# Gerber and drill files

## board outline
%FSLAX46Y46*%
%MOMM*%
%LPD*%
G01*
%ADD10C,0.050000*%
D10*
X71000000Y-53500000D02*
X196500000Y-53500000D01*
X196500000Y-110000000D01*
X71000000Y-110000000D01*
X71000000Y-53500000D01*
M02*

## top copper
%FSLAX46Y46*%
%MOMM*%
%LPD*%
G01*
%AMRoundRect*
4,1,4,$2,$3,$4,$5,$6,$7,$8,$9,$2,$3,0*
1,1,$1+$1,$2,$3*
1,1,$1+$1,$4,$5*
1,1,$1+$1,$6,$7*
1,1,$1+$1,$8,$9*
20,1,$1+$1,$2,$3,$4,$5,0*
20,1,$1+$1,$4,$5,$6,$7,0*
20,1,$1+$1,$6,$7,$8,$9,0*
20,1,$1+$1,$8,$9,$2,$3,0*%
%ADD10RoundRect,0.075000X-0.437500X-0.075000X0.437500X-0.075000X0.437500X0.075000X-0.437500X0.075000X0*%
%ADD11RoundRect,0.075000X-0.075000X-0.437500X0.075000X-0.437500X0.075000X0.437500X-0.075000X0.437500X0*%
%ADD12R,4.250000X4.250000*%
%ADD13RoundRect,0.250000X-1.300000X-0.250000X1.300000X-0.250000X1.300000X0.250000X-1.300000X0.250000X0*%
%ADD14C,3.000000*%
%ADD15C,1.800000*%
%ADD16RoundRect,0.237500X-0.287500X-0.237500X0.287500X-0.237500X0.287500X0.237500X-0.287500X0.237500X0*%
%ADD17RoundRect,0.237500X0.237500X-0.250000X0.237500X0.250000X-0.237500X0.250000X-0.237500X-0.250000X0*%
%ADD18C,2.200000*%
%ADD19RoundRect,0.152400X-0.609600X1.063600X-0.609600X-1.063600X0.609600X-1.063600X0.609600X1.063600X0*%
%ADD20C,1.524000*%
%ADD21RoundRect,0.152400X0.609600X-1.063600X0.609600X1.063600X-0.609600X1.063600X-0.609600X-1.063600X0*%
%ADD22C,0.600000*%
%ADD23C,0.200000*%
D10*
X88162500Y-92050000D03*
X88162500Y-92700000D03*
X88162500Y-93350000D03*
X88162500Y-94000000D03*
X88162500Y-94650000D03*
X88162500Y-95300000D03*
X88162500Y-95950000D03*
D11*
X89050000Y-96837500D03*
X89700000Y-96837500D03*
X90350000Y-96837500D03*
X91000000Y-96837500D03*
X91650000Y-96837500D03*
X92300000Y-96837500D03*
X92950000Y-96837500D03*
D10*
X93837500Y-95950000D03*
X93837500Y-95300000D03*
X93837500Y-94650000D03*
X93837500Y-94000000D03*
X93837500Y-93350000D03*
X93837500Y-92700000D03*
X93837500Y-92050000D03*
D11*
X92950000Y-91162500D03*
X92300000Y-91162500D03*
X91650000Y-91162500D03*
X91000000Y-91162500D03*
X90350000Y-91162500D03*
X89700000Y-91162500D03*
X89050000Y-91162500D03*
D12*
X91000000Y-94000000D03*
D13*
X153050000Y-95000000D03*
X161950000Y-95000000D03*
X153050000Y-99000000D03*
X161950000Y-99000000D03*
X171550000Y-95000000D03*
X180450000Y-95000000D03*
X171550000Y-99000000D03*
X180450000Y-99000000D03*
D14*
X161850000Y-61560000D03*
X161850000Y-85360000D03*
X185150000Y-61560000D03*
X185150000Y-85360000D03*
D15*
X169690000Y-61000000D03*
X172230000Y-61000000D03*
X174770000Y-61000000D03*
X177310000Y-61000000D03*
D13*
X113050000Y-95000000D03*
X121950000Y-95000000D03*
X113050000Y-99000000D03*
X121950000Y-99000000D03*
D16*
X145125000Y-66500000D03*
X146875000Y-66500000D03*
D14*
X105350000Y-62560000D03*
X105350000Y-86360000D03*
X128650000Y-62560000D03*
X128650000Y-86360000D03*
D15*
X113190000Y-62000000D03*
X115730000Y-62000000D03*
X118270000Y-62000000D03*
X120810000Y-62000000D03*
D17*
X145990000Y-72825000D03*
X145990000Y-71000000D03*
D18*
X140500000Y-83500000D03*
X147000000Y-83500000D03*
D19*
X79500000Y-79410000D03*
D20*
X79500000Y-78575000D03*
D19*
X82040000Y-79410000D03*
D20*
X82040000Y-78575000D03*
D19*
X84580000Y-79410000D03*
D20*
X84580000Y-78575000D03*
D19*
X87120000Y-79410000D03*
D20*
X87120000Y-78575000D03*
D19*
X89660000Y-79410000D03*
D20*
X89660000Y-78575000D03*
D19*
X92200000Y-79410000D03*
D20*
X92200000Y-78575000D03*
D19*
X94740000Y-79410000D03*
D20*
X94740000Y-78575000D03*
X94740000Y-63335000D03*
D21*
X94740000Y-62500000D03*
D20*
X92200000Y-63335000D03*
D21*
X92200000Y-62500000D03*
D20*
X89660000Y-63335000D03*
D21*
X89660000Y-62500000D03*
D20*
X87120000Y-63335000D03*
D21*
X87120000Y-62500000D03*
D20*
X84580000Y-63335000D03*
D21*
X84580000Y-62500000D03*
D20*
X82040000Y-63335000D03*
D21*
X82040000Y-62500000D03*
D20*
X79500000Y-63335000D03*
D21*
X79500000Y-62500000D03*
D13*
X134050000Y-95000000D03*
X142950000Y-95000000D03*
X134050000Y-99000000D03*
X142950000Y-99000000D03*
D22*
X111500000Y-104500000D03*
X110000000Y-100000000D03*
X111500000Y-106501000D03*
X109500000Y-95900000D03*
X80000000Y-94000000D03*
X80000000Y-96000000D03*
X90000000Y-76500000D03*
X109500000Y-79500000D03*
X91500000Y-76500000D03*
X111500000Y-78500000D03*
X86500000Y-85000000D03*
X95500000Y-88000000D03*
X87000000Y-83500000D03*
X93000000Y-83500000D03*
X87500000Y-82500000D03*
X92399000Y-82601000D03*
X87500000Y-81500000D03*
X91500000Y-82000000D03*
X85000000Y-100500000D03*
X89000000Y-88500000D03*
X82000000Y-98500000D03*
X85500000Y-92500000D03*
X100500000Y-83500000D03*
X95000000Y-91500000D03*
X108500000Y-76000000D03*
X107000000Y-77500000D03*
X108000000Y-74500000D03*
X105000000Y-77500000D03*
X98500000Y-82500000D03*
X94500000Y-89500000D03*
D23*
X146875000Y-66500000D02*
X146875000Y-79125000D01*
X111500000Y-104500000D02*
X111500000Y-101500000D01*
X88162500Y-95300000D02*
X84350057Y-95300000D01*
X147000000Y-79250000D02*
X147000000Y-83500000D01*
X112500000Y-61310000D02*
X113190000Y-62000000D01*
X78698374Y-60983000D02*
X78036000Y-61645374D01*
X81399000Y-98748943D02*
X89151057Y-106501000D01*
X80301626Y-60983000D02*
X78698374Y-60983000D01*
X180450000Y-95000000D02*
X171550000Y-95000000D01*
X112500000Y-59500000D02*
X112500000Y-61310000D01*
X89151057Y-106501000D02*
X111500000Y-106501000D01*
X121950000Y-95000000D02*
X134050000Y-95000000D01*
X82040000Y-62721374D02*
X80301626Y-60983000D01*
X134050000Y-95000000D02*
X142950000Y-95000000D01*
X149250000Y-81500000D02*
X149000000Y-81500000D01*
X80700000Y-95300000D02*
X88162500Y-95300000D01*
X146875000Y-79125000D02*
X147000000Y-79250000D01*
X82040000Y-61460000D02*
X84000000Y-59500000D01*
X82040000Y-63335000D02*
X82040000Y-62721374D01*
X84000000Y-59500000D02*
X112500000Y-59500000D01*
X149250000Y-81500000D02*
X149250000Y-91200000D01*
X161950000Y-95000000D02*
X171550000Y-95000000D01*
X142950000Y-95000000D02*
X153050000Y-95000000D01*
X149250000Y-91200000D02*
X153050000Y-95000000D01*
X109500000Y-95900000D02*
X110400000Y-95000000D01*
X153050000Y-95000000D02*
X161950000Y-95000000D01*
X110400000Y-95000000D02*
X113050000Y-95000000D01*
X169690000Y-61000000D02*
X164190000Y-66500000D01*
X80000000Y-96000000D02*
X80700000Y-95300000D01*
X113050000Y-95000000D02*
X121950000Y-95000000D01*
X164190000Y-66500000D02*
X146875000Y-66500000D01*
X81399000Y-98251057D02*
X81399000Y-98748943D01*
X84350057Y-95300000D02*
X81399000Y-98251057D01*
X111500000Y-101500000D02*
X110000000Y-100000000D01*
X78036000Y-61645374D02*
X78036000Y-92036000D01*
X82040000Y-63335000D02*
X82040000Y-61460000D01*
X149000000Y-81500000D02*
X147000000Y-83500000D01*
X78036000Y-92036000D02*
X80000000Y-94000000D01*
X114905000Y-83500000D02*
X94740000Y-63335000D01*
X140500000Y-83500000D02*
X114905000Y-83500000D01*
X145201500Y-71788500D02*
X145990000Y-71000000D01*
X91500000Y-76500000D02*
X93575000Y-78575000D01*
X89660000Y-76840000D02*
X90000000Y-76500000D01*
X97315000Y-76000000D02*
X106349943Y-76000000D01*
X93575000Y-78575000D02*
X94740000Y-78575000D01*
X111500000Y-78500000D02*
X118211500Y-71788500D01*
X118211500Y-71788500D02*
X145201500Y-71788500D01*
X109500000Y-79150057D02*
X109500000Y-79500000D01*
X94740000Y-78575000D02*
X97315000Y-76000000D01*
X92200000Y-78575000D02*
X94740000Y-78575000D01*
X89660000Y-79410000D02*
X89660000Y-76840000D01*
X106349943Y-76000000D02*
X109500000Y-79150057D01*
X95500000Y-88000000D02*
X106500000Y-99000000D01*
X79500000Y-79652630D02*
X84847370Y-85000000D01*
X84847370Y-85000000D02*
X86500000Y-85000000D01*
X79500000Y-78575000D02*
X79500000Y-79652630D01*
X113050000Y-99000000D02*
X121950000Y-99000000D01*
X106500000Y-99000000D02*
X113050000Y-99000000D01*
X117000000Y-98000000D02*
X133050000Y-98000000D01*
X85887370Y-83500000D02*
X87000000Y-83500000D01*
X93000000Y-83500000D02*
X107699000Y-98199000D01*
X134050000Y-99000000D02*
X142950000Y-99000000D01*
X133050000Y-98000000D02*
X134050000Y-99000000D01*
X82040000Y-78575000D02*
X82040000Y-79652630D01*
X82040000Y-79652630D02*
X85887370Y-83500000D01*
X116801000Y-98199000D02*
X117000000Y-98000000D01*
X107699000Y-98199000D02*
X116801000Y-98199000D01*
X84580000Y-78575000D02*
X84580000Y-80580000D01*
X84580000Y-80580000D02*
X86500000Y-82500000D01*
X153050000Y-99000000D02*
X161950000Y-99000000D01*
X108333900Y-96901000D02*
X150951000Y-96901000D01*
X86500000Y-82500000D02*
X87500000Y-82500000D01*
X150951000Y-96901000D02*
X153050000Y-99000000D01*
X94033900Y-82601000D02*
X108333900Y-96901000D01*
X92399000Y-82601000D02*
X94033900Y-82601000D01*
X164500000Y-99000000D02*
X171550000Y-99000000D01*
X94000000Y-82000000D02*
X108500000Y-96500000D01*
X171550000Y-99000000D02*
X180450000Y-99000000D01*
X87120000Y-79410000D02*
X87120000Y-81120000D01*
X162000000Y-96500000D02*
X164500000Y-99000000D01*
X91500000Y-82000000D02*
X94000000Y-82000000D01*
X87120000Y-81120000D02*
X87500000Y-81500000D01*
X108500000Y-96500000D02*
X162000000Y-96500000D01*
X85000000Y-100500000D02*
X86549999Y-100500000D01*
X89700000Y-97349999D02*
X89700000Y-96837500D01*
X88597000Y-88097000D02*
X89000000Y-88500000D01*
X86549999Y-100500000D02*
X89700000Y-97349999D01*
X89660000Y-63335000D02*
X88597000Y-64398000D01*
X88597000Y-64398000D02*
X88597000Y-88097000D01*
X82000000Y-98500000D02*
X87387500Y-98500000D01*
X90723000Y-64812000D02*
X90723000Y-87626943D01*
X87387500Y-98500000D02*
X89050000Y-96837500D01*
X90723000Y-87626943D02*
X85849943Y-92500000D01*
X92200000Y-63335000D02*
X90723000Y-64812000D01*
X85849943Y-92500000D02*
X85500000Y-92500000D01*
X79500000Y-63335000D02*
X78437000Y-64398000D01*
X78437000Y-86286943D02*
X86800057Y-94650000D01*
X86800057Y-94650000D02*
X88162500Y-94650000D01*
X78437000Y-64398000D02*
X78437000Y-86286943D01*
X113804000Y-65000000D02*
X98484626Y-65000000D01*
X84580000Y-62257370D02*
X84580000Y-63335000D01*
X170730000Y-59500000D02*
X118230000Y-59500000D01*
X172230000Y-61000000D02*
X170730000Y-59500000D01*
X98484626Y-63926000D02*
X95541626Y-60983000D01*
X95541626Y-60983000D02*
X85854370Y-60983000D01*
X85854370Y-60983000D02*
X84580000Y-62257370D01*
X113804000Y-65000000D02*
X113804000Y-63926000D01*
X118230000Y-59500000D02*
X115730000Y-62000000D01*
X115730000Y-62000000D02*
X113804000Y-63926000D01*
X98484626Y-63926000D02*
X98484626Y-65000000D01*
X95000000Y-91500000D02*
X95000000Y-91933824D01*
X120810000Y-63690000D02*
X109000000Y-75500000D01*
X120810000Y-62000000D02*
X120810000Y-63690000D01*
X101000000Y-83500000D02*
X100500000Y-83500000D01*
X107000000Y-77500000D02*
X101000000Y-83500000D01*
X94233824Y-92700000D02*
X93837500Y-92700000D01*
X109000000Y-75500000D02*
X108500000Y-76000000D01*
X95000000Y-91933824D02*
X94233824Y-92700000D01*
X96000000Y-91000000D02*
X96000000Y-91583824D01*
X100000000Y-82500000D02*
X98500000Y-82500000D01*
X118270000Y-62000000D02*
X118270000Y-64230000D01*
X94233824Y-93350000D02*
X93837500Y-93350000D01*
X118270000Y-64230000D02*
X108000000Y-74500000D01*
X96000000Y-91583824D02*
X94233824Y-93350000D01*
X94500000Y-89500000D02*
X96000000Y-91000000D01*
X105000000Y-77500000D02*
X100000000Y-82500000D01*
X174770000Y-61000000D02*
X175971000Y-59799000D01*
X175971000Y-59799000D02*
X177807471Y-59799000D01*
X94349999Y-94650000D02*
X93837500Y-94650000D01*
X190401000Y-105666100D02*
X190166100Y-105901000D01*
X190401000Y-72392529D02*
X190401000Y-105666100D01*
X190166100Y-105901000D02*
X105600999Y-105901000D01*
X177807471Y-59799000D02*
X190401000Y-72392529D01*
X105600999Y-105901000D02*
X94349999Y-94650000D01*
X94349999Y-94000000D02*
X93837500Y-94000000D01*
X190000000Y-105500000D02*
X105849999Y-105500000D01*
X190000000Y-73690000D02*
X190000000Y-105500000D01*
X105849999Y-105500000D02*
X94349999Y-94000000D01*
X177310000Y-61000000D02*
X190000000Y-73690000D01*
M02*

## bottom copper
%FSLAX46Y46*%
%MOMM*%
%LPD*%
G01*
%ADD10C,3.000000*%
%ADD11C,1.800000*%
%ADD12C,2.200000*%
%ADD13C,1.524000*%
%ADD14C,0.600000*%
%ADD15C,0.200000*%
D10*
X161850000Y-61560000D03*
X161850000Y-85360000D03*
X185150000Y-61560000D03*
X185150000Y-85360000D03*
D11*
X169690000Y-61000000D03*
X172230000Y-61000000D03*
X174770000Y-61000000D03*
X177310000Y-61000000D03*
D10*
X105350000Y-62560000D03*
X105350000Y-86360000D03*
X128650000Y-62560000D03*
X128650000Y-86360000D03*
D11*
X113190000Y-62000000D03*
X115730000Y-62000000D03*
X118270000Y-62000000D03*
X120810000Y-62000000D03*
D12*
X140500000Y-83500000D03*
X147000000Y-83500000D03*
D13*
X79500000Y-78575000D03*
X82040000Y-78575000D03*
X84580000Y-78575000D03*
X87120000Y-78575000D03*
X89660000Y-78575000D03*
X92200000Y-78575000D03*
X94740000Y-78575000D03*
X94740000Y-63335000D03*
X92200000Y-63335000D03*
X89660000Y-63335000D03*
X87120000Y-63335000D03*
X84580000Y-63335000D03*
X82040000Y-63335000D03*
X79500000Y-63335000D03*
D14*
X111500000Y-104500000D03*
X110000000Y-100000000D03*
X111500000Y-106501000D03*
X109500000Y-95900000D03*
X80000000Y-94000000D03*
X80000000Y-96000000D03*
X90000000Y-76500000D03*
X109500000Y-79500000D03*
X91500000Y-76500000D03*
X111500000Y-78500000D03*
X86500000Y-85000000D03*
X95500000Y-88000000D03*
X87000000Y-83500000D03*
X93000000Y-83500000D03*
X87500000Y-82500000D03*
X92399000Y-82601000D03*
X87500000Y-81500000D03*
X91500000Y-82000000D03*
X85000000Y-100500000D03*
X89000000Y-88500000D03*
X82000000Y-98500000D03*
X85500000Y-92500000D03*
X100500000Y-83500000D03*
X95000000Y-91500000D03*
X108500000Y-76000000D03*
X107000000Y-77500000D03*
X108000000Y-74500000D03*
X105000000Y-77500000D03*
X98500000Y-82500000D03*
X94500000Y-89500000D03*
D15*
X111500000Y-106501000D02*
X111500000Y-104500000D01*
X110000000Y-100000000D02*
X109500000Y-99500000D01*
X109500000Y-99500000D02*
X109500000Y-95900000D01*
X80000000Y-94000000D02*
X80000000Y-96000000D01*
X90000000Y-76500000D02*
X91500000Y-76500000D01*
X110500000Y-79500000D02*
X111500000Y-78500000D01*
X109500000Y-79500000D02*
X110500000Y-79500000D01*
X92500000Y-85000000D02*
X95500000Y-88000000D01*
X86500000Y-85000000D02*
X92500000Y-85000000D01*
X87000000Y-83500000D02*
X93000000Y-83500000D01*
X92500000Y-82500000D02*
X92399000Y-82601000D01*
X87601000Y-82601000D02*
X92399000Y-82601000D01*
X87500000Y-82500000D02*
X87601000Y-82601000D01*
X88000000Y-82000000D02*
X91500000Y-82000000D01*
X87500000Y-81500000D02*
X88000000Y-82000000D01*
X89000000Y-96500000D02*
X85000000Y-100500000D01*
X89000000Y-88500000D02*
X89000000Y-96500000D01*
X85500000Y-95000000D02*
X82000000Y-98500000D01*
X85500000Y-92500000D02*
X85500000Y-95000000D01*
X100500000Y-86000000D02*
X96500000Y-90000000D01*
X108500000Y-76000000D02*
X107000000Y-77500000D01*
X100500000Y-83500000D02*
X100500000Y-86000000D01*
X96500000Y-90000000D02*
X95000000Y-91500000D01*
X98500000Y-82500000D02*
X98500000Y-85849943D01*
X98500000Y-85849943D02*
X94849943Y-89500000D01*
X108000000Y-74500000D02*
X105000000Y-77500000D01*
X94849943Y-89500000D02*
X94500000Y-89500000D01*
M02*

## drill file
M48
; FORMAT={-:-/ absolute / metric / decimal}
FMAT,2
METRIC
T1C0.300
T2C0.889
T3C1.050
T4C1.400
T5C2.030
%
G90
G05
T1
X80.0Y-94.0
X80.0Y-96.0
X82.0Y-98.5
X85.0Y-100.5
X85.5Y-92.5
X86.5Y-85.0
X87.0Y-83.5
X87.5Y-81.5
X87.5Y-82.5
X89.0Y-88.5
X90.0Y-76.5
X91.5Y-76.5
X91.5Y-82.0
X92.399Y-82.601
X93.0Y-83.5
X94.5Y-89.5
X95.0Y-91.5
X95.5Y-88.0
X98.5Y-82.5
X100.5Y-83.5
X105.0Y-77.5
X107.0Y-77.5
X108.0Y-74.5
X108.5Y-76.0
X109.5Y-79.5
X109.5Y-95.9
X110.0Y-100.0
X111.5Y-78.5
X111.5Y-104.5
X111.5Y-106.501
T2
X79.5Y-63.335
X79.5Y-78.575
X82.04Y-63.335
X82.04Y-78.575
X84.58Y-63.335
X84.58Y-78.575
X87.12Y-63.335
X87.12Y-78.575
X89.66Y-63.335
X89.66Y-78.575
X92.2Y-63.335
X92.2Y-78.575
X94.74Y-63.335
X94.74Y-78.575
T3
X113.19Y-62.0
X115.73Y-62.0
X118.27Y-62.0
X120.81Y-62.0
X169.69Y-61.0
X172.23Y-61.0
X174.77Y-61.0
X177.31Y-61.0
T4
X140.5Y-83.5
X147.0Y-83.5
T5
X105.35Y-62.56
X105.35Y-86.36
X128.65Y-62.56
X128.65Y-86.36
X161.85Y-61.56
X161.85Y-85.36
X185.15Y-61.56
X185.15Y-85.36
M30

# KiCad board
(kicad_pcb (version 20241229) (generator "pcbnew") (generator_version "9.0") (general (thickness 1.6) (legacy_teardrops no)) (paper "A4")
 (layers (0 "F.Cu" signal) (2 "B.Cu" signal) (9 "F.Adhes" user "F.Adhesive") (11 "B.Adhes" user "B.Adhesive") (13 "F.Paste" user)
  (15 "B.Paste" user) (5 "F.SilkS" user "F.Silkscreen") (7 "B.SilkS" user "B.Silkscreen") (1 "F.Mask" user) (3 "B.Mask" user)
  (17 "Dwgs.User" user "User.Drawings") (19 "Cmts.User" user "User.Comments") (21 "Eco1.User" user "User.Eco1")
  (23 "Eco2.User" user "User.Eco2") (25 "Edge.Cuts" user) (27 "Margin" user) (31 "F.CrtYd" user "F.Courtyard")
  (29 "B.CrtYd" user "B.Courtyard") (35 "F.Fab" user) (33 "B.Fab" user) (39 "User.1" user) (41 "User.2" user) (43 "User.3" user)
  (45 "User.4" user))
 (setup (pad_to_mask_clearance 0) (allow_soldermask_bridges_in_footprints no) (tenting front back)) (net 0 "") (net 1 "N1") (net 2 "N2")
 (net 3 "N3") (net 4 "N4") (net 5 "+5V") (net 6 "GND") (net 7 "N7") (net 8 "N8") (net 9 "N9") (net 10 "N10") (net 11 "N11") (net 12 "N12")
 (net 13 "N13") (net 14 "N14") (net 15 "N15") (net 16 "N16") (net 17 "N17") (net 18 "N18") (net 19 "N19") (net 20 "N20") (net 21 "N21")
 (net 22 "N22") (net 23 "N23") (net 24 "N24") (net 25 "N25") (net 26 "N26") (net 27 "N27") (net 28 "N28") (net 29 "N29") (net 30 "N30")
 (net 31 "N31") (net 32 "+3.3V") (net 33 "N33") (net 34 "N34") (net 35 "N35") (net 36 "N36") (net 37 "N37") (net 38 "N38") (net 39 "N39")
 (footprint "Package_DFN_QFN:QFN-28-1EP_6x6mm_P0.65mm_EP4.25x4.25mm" (layer "F.Cu") (at 91 94)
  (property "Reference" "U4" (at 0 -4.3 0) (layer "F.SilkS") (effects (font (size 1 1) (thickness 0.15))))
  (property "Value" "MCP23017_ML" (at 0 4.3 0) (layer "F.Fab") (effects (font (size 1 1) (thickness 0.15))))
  (pad "" smd roundrect (at -1.42 -1.42) (size 1.14 1.14) (layers "F.Paste") (roundrect_rratio 0.219298))
  (pad "" smd roundrect (at -1.42 0) (size 1.14 1.14) (layers "F.Paste") (roundrect_rratio 0.219298))
  (pad "" smd roundrect (at -1.42 1.42) (size 1.14 1.14) (layers "F.Paste") (roundrect_rratio 0.219298))
  (pad "" smd roundrect (at 0 -1.42) (size 1.14 1.14) (layers "F.Paste") (roundrect_rratio 0.219298))
  (pad "" smd roundrect (at 0 0) (size 1.14 1.14) (layers "F.Paste") (roundrect_rratio 0.219298))
  (pad "" smd roundrect (at 0 1.42) (size 1.14 1.14) (layers "F.Paste") (roundrect_rratio 0.219298))
  (pad "" smd roundrect (at 1.42 -1.42) (size 1.14 1.14) (layers "F.Paste") (roundrect_rratio 0.219298))
  (pad "" smd roundrect (at 1.42 0) (size 1.14 1.14) (layers "F.Paste") (roundrect_rratio 0.219298))
  (pad "" smd roundrect (at 1.42 1.42) (size 1.14 1.14) (layers "F.Paste") (roundrect_rratio 0.219298))
  (pad "1" smd roundrect (at -2.8375 -1.95) (size 1.025 0.3) (layers "F.Cu" "F.Mask" "F.Paste") (roundrect_rratio 0.25) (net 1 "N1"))
  (pad "2" smd roundrect (at -2.8375 -1.3) (size 1.025 0.3) (layers "F.Cu" "F.Mask" "F.Paste") (roundrect_rratio 0.25) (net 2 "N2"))
  (pad "3" smd roundrect (at -2.8375 -0.65) (size 1.025 0.3) (layers "F.Cu" "F.Mask" "F.Paste") (roundrect_rratio 0.25) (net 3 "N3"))
  (pad "4" smd roundrect (at -2.8375 0) (size 1.025 0.3) (layers "F.Cu" "F.Mask" "F.Paste") (roundrect_rratio 0.25) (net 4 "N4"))
  (pad "5" smd roundrect (at -2.8375 0.65) (size 1.025 0.3) (layers "F.Cu" "F.Mask" "F.Paste") (roundrect_rratio 0.25) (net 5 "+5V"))
  (pad "6" smd roundrect (at -2.8375 1.3) (size 1.025 0.3) (layers "F.Cu" "F.Mask" "F.Paste") (roundrect_rratio 0.25) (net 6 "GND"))
  (pad "7" smd roundrect (at -2.8375 1.95) (size 1.025 0.3) (layers "F.Cu" "F.Mask" "F.Paste") (roundrect_rratio 0.25) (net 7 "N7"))
  (pad "8" smd roundrect (at -1.95 2.8375) (size 0.3 1.025) (layers "F.Cu" "F.Mask" "F.Paste") (roundrect_rratio 0.25) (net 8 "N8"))
  (pad "9" smd roundrect (at -1.3 2.8375) (size 0.3 1.025) (layers "F.Cu" "F.Mask" "F.Paste") (roundrect_rratio 0.25) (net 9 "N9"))
  (pad "10" smd roundrect (at -0.65 2.8375) (size 0.3 1.025) (layers "F.Cu" "F.Mask" "F.Paste") (roundrect_rratio 0.25) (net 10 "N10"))
  (pad "11" smd roundrect (at 0 2.8375) (size 0.3 1.025) (layers "F.Cu" "F.Mask" "F.Paste") (roundrect_rratio 0.25) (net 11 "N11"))
  (pad "12" smd roundrect (at 0.65 2.8375) (size 0.3 1.025) (layers "F.Cu" "F.Mask" "F.Paste") (roundrect_rratio 0.25) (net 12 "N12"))
  (pad "13" smd roundrect (at 1.3 2.8375) (size 0.3 1.025) (layers "F.Cu" "F.Mask" "F.Paste") (roundrect_rratio 0.25) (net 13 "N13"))
  (pad "14" smd roundrect (at 1.95 2.8375) (size 0.3 1.025) (layers "F.Cu" "F.Mask" "F.Paste") (roundrect_rratio 0.25) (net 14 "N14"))
  (pad "15" smd roundrect (at 2.8375 1.95) (size 1.025 0.3) (layers "F.Cu" "F.Mask" "F.Paste") (roundrect_rratio 0.25) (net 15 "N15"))
  (pad "16" smd roundrect (at 2.8375 1.3) (size 1.025 0.3) (layers "F.Cu" "F.Mask" "F.Paste") (roundrect_rratio 0.25) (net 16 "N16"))
  (pad "17" smd roundrect (at 2.8375 0.65) (size 1.025 0.3) (layers "F.Cu" "F.Mask" "F.Paste") (roundrect_rratio 0.25) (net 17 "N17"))
  (pad "18" smd roundrect (at 2.8375 0) (size 1.025 0.3) (layers "F.Cu" "F.Mask" "F.Paste") (roundrect_rratio 0.25) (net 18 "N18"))
  (pad "19" smd roundrect (at 2.8375 -0.65) (size 1.025 0.3) (layers "F.Cu" "F.Mask" "F.Paste") (roundrect_rratio 0.25) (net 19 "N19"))
  (pad "20" smd roundrect (at 2.8375 -1.3) (size 1.025 0.3) (layers "F.Cu" "F.Mask" "F.Paste") (roundrect_rratio 0.25) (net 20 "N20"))
  (pad "21" smd roundrect (at 2.8375 -1.95) (size 1.025 0.3) (layers "F.Cu" "F.Mask" "F.Paste") (roundrect_rratio 0.25) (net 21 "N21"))
  (pad "22" smd roundrect (at 1.95 -2.8375) (size 0.3 1.025) (layers "F.Cu" "F.Mask" "F.Paste") (roundrect_rratio 0.25) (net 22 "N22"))
  (pad "23" smd roundrect (at 1.3 -2.8375) (size 0.3 1.025) (layers "F.Cu" "F.Mask" "F.Paste") (roundrect_rratio 0.25) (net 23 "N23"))
  (pad "24" smd roundrect (at 0.65 -2.8375) (size 0.3 1.025) (layers "F.Cu" "F.Mask" "F.Paste") (roundrect_rratio 0.25) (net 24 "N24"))
  (pad "25" smd roundrect (at 0 -2.8375) (size 0.3 1.025) (layers "F.Cu" "F.Mask" "F.Paste") (roundrect_rratio 0.25) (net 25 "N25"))
  (pad "26" smd roundrect (at -0.65 -2.8375) (size 0.3 1.025) (layers "F.Cu" "F.Mask" "F.Paste") (roundrect_rratio 0.25) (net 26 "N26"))
  (pad "27" smd roundrect (at -1.3 -2.8375) (size 0.3 1.025) (layers "F.Cu" "F.Mask" "F.Paste") (roundrect_rratio 0.25) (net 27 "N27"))
  (pad "28" smd roundrect (at -1.95 -2.8375) (size 0.3 1.025) (layers "F.Cu" "F.Mask" "F.Paste") (roundrect_rratio 0.25) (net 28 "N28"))
  (pad "29" smd rect (at 0 0) (size 4.25 4.25) (layers "F.Cu" "F.Mask") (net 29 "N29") (zone_connect 2)))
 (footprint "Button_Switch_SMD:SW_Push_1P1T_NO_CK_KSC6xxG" (layer "F.Cu") (at 157.5 97)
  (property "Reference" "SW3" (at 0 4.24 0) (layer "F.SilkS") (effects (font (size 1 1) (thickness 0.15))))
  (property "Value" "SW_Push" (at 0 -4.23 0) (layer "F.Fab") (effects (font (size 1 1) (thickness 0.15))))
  (pad "1" smd roundrect (at -4.45 -2) (size 3.1 1) (layers "F.Cu" "F.Mask" "F.Paste") (roundrect_rratio 0.25) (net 6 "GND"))
  (pad "1" smd roundrect (at 4.45 -2) (size 3.1 1) (layers "F.Cu" "F.Mask" "F.Paste") (roundrect_rratio 0.25) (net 6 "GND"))
  (pad "2" smd roundrect (at -4.45 2) (size 3.1 1) (layers "F.Cu" "F.Mask" "F.Paste") (roundrect_rratio 0.25) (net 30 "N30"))
  (pad "2" smd roundrect (at 4.45 2) (size 3.1 1) (layers "F.Cu" "F.Mask" "F.Paste") (roundrect_rratio 0.25) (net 30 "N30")))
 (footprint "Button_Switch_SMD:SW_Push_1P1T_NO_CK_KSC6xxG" (layer "F.Cu") (at 176 97)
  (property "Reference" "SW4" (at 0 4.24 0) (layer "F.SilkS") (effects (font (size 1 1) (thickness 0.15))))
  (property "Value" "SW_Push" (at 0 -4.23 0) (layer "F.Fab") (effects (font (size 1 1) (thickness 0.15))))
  (pad "1" smd roundrect (at -4.45 -2) (size 3.1 1) (layers "F.Cu" "F.Mask" "F.Paste") (roundrect_rratio 0.25) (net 6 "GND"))
  (pad "1" smd roundrect (at 4.45 -2) (size 3.1 1) (layers "F.Cu" "F.Mask" "F.Paste") (roundrect_rratio 0.25) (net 6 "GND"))
  (pad "2" smd roundrect (at -4.45 2) (size 3.1 1) (layers "F.Cu" "F.Mask" "F.Paste") (roundrect_rratio 0.25) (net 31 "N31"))
  (pad "2" smd roundrect (at 4.45 2) (size 3.1 1) (layers "F.Cu" "F.Mask" "F.Paste") (roundrect_rratio 0.25) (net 31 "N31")))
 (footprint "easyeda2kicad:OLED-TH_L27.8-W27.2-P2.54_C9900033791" (layer "F.Cu") (at 173.5 61)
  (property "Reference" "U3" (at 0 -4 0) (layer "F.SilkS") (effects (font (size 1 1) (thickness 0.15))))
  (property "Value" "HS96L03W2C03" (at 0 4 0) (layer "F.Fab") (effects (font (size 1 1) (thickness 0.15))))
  (pad "" thru_hole circle (at -11.65 0.56) (size 3 3) (drill 2.03) (layers "*.Cu" "*.Mask") (remove_unused_layers no))
  (pad "" thru_hole circle (at -11.65 24.36) (size 3 3) (drill 2.03) (layers "*.Cu" "*.Mask") (remove_unused_layers no))
  (pad "" thru_hole circle (at 11.65 0.56) (size 3 3) (drill 2.03) (layers "*.Cu" "*.Mask") (remove_unused_layers no))
  (pad "" thru_hole circle (at 11.65 24.36) (size 3 3) (drill 2.03) (layers "*.Cu" "*.Mask") (remove_unused_layers no))
  (pad "1" thru_hole circle (at -3.81 0) (size 1.8 1.8) (drill 1.049986) (layers "*.Cu" "*.Mask") (remove_unused_layers no) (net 6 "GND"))
  (pad "2" thru_hole circle (at -1.27 0) (size 1.8 1.8) (drill 1.049986) (layers "*.Cu" "*.Mask") (remove_unused_layers no) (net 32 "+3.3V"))
  (pad "3" thru_hole circle (at 1.27 0) (size 1.8 1.8) (drill 1.049986) (layers "*.Cu" "*.Mask") (remove_unused_layers no) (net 17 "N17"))
  (pad "4" thru_hole circle (at 3.81 0) (size 1.8 1.8) (drill 1.049986) (layers "*.Cu" "*.Mask") (remove_unused_layers no) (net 18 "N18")))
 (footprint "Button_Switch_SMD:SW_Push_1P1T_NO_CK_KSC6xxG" (layer "F.Cu") (at 117.5 97)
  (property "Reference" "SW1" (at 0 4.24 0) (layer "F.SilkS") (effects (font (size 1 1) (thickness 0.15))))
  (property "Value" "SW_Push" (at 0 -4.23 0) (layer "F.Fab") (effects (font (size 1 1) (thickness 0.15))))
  (pad "1" smd roundrect (at -4.45 -2) (size 3.1 1) (layers "F.Cu" "F.Mask" "F.Paste") (roundrect_rratio 0.25) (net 6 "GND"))
  (pad "1" smd roundrect (at 4.45 -2) (size 3.1 1) (layers "F.Cu" "F.Mask" "F.Paste") (roundrect_rratio 0.25) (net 6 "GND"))
  (pad "2" smd roundrect (at -4.45 2) (size 3.1 1) (layers "F.Cu" "F.Mask" "F.Paste") (roundrect_rratio 0.25) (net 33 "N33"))
  (pad "2" smd roundrect (at 4.45 2) (size 3.1 1) (layers "F.Cu" "F.Mask" "F.Paste") (roundrect_rratio 0.25) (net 33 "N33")))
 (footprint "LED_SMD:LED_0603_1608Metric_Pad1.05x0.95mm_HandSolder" (layer "F.Cu") (at 146 66.5)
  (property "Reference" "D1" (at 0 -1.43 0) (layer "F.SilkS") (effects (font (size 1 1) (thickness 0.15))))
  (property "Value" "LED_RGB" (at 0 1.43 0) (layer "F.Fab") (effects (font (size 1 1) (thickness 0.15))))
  (pad "1" smd roundrect (at -0.875 0) (size 1.05 0.95) (layers "F.Cu" "F.Mask" "F.Paste") (roundrect_rratio 0.25) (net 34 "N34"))
  (pad "2" smd roundrect (at 0.875 0) (size 1.05 0.95) (layers "F.Cu" "F.Mask" "F.Paste") (roundrect_rratio 0.25) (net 6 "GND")))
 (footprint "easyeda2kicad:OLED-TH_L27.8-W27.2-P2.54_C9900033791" (layer "F.Cu") (at 117 62)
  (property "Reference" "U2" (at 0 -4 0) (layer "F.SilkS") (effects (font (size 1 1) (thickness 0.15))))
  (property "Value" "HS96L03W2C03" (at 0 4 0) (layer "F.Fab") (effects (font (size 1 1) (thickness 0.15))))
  (pad "" thru_hole circle (at -11.65 0.56) (size 3 3) (drill 2.03) (layers "*.Cu" "*.Mask") (remove_unused_layers no))
  (pad "" thru_hole circle (at -11.65 24.36) (size 3 3) (drill 2.03) (layers "*.Cu" "*.Mask") (remove_unused_layers no))
  (pad "" thru_hole circle (at 11.65 0.56) (size 3 3) (drill 2.03) (layers "*.Cu" "*.Mask") (remove_unused_layers no))
  (pad "" thru_hole circle (at 11.65 24.36) (size 3 3) (drill 2.03) (layers "*.Cu" "*.Mask") (remove_unused_layers no))
  (pad "1" thru_hole circle (at -3.81 0) (size 1.8 1.8) (drill 1.049986) (layers "*.Cu" "*.Mask") (remove_unused_layers no) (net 6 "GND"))
  (pad "2" thru_hole circle (at -1.27 0) (size 1.8 1.8) (drill 1.049986) (layers "*.Cu" "*.Mask") (remove_unused_layers no) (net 32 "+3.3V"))
  (pad "3" thru_hole circle (at 1.27 0) (size 1.8 1.8) (drill 1.049986) (layers "*.Cu" "*.Mask") (remove_unused_layers no) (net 19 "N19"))
  (pad "4" thru_hole circle (at 3.81 0) (size 1.8 1.8) (drill 1.049986) (layers "*.Cu" "*.Mask") (remove_unused_layers no) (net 20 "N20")))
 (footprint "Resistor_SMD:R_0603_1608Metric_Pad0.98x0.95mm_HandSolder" (layer "F.Cu") (at 145.99 71.9125 90)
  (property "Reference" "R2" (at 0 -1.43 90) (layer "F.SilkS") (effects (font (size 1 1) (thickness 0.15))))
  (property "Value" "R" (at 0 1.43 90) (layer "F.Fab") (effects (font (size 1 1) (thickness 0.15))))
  (pad "1" smd roundrect (at -0.9125 0 90) (size 0.975 0.95) (layers "F.Cu" "F.Mask" "F.Paste") (roundrect_rratio 0.25) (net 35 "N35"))
  (pad "2" smd roundrect (at 0.9125 0 90) (size 0.975 0.95) (layers "F.Cu" "F.Mask" "F.Paste") (roundrect_rratio 0.25) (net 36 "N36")))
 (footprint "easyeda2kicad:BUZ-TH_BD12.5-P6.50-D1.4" (layer "F.Cu") (at 143.75 83.5)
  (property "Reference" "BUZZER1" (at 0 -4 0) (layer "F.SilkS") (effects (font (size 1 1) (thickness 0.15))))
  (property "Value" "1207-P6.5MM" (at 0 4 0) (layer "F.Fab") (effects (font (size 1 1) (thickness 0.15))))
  (pad "1" thru_hole circle (at -3.25 0) (size 2.2 2.2) (drill 1.399998) (layers "*.Cu" "*.Mask") (remove_unused_layers no) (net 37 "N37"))
  (pad "2" thru_hole circle (at 3.25 0) (size 2.2 2.2) (drill 1.399998) (layers "*.Cu" "*.Mask") (remove_unused_layers no) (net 6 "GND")))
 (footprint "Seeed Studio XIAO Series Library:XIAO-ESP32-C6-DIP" (layer "F.Cu") (at 87.12 70.955 180)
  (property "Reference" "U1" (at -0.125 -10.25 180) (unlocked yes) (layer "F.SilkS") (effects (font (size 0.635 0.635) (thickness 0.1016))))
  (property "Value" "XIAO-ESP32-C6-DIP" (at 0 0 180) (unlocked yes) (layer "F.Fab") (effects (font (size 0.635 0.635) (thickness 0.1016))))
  (pad "1" smd roundrect (at 7.62 -8.455 270) (size 2.432 1.524) (layers "F.Cu" "F.Mask") (roundrect_rratio 0.1) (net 33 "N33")
   (thermal_bridge_angle 45))
  (pad "1" thru_hole circle (at 7.62 -7.62 270) (size 1.524 1.524) (drill 0.889) (layers "*.Cu" "*.Mask") (remove_unused_layers no)
   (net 33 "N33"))
  (pad "2" smd roundrect (at 5.08 -8.455 270) (size 2.432 1.524) (layers "F.Cu" "F.Mask") (roundrect_rratio 0.1) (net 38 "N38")
   (thermal_bridge_angle 45))
  (pad "2" thru_hole circle (at 5.08 -7.62 270) (size 1.524 1.524) (drill 0.889) (layers "*.Cu" "*.Mask") (remove_unused_layers no)
   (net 38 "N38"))
  (pad "3" smd roundrect (at 2.54 -8.455 270) (size 2.432 1.524) (layers "F.Cu" "F.Mask") (roundrect_rratio 0.1) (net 30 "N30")
   (thermal_bridge_angle 45))
  (pad "3" thru_hole circle (at 2.54 -7.62 270) (size 1.524 1.524) (drill 0.889) (layers "*.Cu" "*.Mask") (remove_unused_layers no)
   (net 30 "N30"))
  (pad "4" smd roundrect (at 0 -8.455 270) (size 2.432 1.524) (layers "F.Cu" "F.Mask") (roundrect_rratio 0.1) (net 31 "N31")
   (thermal_bridge_angle 45))
  (pad "4" thru_hole circle (at 0 -7.62 270) (size 1.524 1.524) (drill 0.889) (layers "*.Cu" "*.Mask") (remove_unused_layers no)
   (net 31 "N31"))
  (pad "5" smd roundrect (at -2.54 -8.455 270) (size 2.432 1.524) (layers "F.Cu" "F.Mask") (roundrect_rratio 0.1) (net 36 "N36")
   (thermal_bridge_angle 45))
  (pad "5" thru_hole circle (at -2.54 -7.62 270) (size 1.524 1.524) (drill 0.889) (layers "*.Cu" "*.Mask") (remove_unused_layers no)
   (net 36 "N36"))
  (pad "6" smd roundrect (at -5.08 -8.455 270) (size 2.432 1.524) (layers "F.Cu" "F.Mask") (roundrect_rratio 0.1) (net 36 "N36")
   (thermal_bridge_angle 45))
  (pad "6" thru_hole circle (at -5.08 -7.62 270) (size 1.524 1.524) (drill 0.889) (layers "*.Cu" "*.Mask") (remove_unused_layers no)
   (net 36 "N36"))
  (pad "7" smd roundrect (at -7.62 -8.455 270) (size 2.432 1.524) (layers "F.Cu" "F.Mask") (roundrect_rratio 0.1) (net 36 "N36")
   (thermal_bridge_angle 45))
  (pad "7" thru_hole circle (at -7.62 -7.62 270) (size 1.524 1.524) (drill 0.889) (layers "*.Cu" "*.Mask") (remove_unused_layers no)
   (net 36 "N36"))
  (pad "8" thru_hole circle (at -7.62 7.62 90) (size 1.524 1.524) (drill 0.889) (layers "*.Cu" "*.Mask") (remove_unused_layers no)
   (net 37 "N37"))
  (pad "8" smd roundrect (at -7.62 8.455 90) (size 2.432 1.524) (layers "F.Cu" "F.Mask") (roundrect_rratio 0.1) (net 37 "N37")
   (thermal_bridge_angle 45))
  (pad "9" thru_hole circle (at -5.08 7.62 90) (size 1.524 1.524) (drill 0.889) (layers "*.Cu" "*.Mask") (remove_unused_layers no)
   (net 8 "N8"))
  (pad "9" smd roundrect (at -5.08 8.455 90) (size 2.432 1.524) (layers "F.Cu" "F.Mask") (roundrect_rratio 0.1) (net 8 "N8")
   (thermal_bridge_angle 45))
  (pad "10" thru_hole circle (at -2.54 7.62 90) (size 1.524 1.524) (drill 0.889) (layers "*.Cu" "*.Mask") (remove_unused_layers no)
   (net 9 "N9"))
  (pad "10" smd roundrect (at -2.54 8.455 90) (size 2.432 1.524) (layers "F.Cu" "F.Mask") (roundrect_rratio 0.1) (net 9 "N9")
   (thermal_bridge_angle 45))
  (pad "11" thru_hole circle (at 0 7.62 90) (size 1.524 1.524) (drill 0.889) (layers "*.Cu" "*.Mask") (remove_unused_layers no)
   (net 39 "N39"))
  (pad "11" smd roundrect (at 0 8.455 90) (size 2.432 1.524) (layers "F.Cu" "F.Mask") (roundrect_rratio 0.1) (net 39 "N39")
   (thermal_bridge_angle 45))
  (pad "12" thru_hole circle (at 2.54 7.62 90) (size 1.524 1.524) (drill 0.889) (layers "*.Cu" "*.Mask") (remove_unused_layers no)
   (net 32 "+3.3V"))
  (pad "12" smd roundrect (at 2.54 8.455 90) (size 2.432 1.524) (layers "F.Cu" "F.Mask") (roundrect_rratio 0.1) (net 32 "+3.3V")
   (thermal_bridge_angle 45))
  (pad "13" thru_hole circle (at 5.08 7.62 90) (size 1.524 1.524) (drill 0.889) (layers "*.Cu" "*.Mask") (remove_unused_layers no)
   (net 6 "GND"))
  (pad "13" smd roundrect (at 5.08 8.455 90) (size 2.432 1.524) (layers "F.Cu" "F.Mask") (roundrect_rratio 0.1) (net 6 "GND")
   (thermal_bridge_angle 45))
  (pad "14" thru_hole circle (at 7.62 7.62 90) (size 1.524 1.524) (drill 0.889) (layers "*.Cu" "*.Mask") (remove_unused_layers no)
   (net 5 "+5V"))
  (pad "14" smd roundrect (at 7.62 8.455 90) (size 2.432 1.524) (layers "F.Cu" "F.Mask") (roundrect_rratio 0.1) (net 5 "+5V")
   (thermal_bridge_angle 45)))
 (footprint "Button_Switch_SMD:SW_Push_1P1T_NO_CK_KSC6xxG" (layer "F.Cu") (at 138.5 97)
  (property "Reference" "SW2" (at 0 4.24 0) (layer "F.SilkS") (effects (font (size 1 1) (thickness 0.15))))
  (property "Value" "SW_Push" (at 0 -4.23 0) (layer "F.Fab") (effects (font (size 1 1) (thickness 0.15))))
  (pad "1" smd roundrect (at -4.45 -2) (size 3.1 1) (layers "F.Cu" "F.Mask" "F.Paste") (roundrect_rratio 0.25) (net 6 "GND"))
  (pad "1" smd roundrect (at 4.45 -2) (size 3.1 1) (layers "F.Cu" "F.Mask" "F.Paste") (roundrect_rratio 0.25) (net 6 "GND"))
  (pad "2" smd roundrect (at -4.45 2) (size 3.1 1) (layers "F.Cu" "F.Mask" "F.Paste") (roundrect_rratio 0.25) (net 38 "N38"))
  (pad "2" smd roundrect (at 4.45 2) (size 3.1 1) (layers "F.Cu" "F.Mask" "F.Paste") (roundrect_rratio 0.25) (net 38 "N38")))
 (gr_rect (start 71 53.5) (end 196.5 110) (stroke (width 0.05) (type default)) (fill no) (layer "Edge.Cuts"))
 (segment (start 146.875 66.5) (end 146.875 79.125) (width 0.2) (layer "F.Cu") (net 6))
 (segment (start 111.5 104.5) (end 111.5 101.5) (width 0.2) (layer "F.Cu") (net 6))
 (segment (start 88.1625 95.3) (end 84.350057 95.3) (width 0.2) (layer "F.Cu") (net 6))
 (segment (start 147 79.25) (end 147 83.5) (width 0.2) (layer "F.Cu") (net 6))
 (segment (start 112.5 61.31) (end 113.19 62) (width 0.2) (layer "F.Cu") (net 6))
 (segment (start 78.698374 60.983) (end 78.036 61.645374) (width 0.2) (layer "F.Cu") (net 6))
 (segment (start 81.399 98.748943) (end 89.151057 106.501) (width 0.2) (layer "F.Cu") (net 6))
 (segment (start 80.301626 60.983) (end 78.698374 60.983) (width 0.2) (layer "F.Cu") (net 6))
 (segment (start 180.45 95) (end 171.55 95) (width 0.2) (layer "F.Cu") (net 6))
 (segment (start 112.5 59.5) (end 112.5 61.31) (width 0.2) (layer "F.Cu") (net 6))
 (segment (start 89.151057 106.501) (end 111.5 106.501) (width 0.2) (layer "F.Cu") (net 6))
 (segment (start 121.95 95) (end 134.05 95) (width 0.2) (layer "F.Cu") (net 6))
 (segment (start 82.04 62.721374) (end 80.301626 60.983) (width 0.2) (layer "F.Cu") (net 6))
 (segment (start 134.05 95) (end 142.95 95) (width 0.2) (layer "F.Cu") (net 6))
 (segment (start 149.25 81.5) (end 149 81.5) (width 0.2) (layer "F.Cu") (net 6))
 (segment (start 80.7 95.3) (end 88.1625 95.3) (width 0.2) (layer "F.Cu") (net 6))
 (segment (start 146.875 79.125) (end 147 79.25) (width 0.2) (layer "F.Cu") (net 6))
 (segment (start 82.04 61.46) (end 84 59.5) (width 0.2) (layer "F.Cu") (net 6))
 (segment (start 82.04 63.335) (end 82.04 62.721374) (width 0.2) (layer "F.Cu") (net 6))
 (segment (start 84 59.5) (end 112.5 59.5) (width 0.2) (layer "F.Cu") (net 6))
 (segment (start 149.25 81.5) (end 149.25 91.2) (width 0.2) (layer "F.Cu") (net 6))
 (segment (start 161.95 95) (end 171.55 95) (width 0.2) (layer "F.Cu") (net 6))
 (segment (start 142.95 95) (end 153.05 95) (width 0.2) (layer "F.Cu") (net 6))
 (segment (start 149.25 91.2) (end 153.05 95) (width 0.2) (layer "F.Cu") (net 6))
 (segment (start 109.5 95.9) (end 110.4 95) (width 0.2) (layer "F.Cu") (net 6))
 (segment (start 153.05 95) (end 161.95 95) (width 0.2) (layer "F.Cu") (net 6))
 (segment (start 110.4 95) (end 113.05 95) (width 0.2) (layer "F.Cu") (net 6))
 (segment (start 169.69 61) (end 164.19 66.5) (width 0.2) (layer "F.Cu") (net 6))
 (segment (start 80 96) (end 80.7 95.3) (width 0.2) (layer "F.Cu") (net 6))
 (segment (start 113.05 95) (end 121.95 95) (width 0.2) (layer "F.Cu") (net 6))
 (segment (start 164.19 66.5) (end 146.875 66.5) (width 0.2) (layer "F.Cu") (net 6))
 (segment (start 81.399 98.251057) (end 81.399 98.748943) (width 0.2) (layer "F.Cu") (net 6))
 (segment (start 84.350057 95.3) (end 81.399 98.251057) (width 0.2) (layer "F.Cu") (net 6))
 (segment (start 111.5 101.5) (end 110 100) (width 0.2) (layer "F.Cu") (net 6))
 (segment (start 78.036 61.645374) (end 78.036 92.036) (width 0.2) (layer "F.Cu") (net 6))
 (segment (start 82.04 63.335) (end 82.04 61.46) (width 0.2) (layer "F.Cu") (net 6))
 (segment (start 149 81.5) (end 147 83.5) (width 0.2) (layer "F.Cu") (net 6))
 (segment (start 78.036 92.036) (end 80 94) (width 0.2) (layer "F.Cu") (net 6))
 (via (at 111.5 104.5) (size 0.6) (drill 0.3) (layers "F.Cu" "B.Cu") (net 6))
 (via (at 110 100) (size 0.6) (drill 0.3) (layers "F.Cu" "B.Cu") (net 6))
 (via (at 111.5 106.501) (size 0.6) (drill 0.3) (layers "F.Cu" "B.Cu") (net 6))
 (via (at 109.5 95.9) (size 0.6) (drill 0.3) (layers "F.Cu" "B.Cu") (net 6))
 (via (at 80 94) (size 0.6) (drill 0.3) (layers "F.Cu" "B.Cu") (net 6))
 (via (at 80 96) (size 0.6) (drill 0.3) (layers "F.Cu" "B.Cu") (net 6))
 (segment (start 111.5 106.501) (end 111.5 104.5) (width 0.2) (layer "B.Cu") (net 6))
 (segment (start 110 100) (end 109.5 99.5) (width 0.2) (layer "B.Cu") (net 6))
 (segment (start 109.5 99.5) (end 109.5 95.9) (width 0.2) (layer "B.Cu") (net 6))
 (segment (start 80 94) (end 80 96) (width 0.2) (layer "B.Cu") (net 6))
 (segment (start 114.905 83.5) (end 94.74 63.335) (width 0.2) (layer "F.Cu") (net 37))
 (segment (start 140.5 83.5) (end 114.905 83.5) (width 0.2) (layer "F.Cu") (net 37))
 (segment (start 145.2015 71.7885) (end 145.99 71) (width 0.2) (layer "F.Cu") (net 36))
 (segment (start 91.5 76.5) (end 93.575 78.575) (width 0.2) (layer "F.Cu") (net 36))
 (segment (start 89.66 76.84) (end 90 76.5) (width 0.2) (layer "F.Cu") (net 36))
 (segment (start 97.315 76) (end 106.349943 76) (width 0.2) (layer "F.Cu") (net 36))
 (segment (start 93.575 78.575) (end 94.74 78.575) (width 0.2) (layer "F.Cu") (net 36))
 (segment (start 111.5 78.5) (end 118.2115 71.7885) (width 0.2) (layer "F.Cu") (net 36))
 (segment (start 118.2115 71.7885) (end 145.2015 71.7885) (width 0.2) (layer "F.Cu") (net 36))
 (segment (start 109.5 79.150057) (end 109.5 79.5) (width 0.2) (layer "F.Cu") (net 36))
 (segment (start 94.74 78.575) (end 97.315 76) (width 0.2) (layer "F.Cu") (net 36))
 (segment (start 92.2 78.575) (end 94.74 78.575) (width 0.2) (layer "F.Cu") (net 36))
 (segment (start 89.66 79.41) (end 89.66 76.84) (width 0.2) (layer "F.Cu") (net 36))
 (segment (start 106.349943 76) (end 109.5 79.150057) (width 0.2) (layer "F.Cu") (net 36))
 (via (at 90 76.5) (size 0.6) (drill 0.3) (layers "F.Cu" "B.Cu") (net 36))
 (via (at 109.5 79.5) (size 0.6) (drill 0.3) (layers "F.Cu" "B.Cu") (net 36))
 (via (at 91.5 76.5) (size 0.6) (drill 0.3) (layers "F.Cu" "B.Cu") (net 36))
 (via (at 111.5 78.5) (size 0.6) (drill 0.3) (layers "F.Cu" "B.Cu") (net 36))
 (segment (start 90 76.5) (end 91.5 76.5) (width 0.2) (layer "B.Cu") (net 36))
 (segment (start 110.5 79.5) (end 111.5 78.5) (width 0.2) (layer "B.Cu") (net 36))
 (segment (start 109.5 79.5) (end 110.5 79.5) (width 0.2) (layer "B.Cu") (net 36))
 (segment (start 95.5 88) (end 106.5 99) (width 0.2) (layer "F.Cu") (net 33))
 (segment (start 79.5 79.65263) (end 84.84737 85) (width 0.2) (layer "F.Cu") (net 33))
 (segment (start 84.84737 85) (end 86.5 85) (width 0.2) (layer "F.Cu") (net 33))
 (segment (start 79.5 78.575) (end 79.5 79.65263) (width 0.2) (layer "F.Cu") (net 33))
 (segment (start 113.05 99) (end 121.95 99) (width 0.2) (layer "F.Cu") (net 33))
 (segment (start 106.5 99) (end 113.05 99) (width 0.2) (layer "F.Cu") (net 33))
 (via (at 86.5 85) (size 0.6) (drill 0.3) (layers "F.Cu" "B.Cu") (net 33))
 (via (at 95.5 88) (size 0.6) (drill 0.3) (layers "F.Cu" "B.Cu") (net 33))
 (segment (start 92.5 85) (end 95.5 88) (width 0.2) (layer "B.Cu") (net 33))
 (segment (start 86.5 85) (end 92.5 85) (width 0.2) (layer "B.Cu") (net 33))
 (segment (start 117 98) (end 133.05 98) (width 0.2) (layer "F.Cu") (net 38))
 (segment (start 85.88737 83.5) (end 87 83.5) (width 0.2) (layer "F.Cu") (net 38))
 (segment (start 93 83.5) (end 107.699 98.199) (width 0.2) (layer "F.Cu") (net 38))
 (segment (start 134.05 99) (end 142.95 99) (width 0.2) (layer "F.Cu") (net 38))
 (segment (start 133.05 98) (end 134.05 99) (width 0.2) (layer "F.Cu") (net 38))
 (segment (start 82.04 78.575) (end 82.04 79.65263) (width 0.2) (layer "F.Cu") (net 38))
 (segment (start 82.04 79.65263) (end 85.88737 83.5) (width 0.2) (layer "F.Cu") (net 38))
 (segment (start 116.801 98.199) (end 117 98) (width 0.2) (layer "F.Cu") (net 38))
 (segment (start 107.699 98.199) (end 116.801 98.199) (width 0.2) (layer "F.Cu") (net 38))
 (via (at 87 83.5) (size 0.6) (drill 0.3) (layers "F.Cu" "B.Cu") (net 38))
 (via (at 93 83.5) (size 0.6) (drill 0.3) (layers "F.Cu" "B.Cu") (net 38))
 (segment (start 87 83.5) (end 93 83.5) (width 0.2) (layer "B.Cu") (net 38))
 (segment (start 84.58 78.575) (end 84.58 80.58) (width 0.2) (layer "F.Cu") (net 30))
 (segment (start 84.58 80.58) (end 86.5 82.5) (width 0.2) (layer "F.Cu") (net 30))
 (segment (start 153.05 99) (end 161.95 99) (width 0.2) (layer "F.Cu") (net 30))
 (segment (start 108.3339 96.901) (end 150.951 96.901) (width 0.2) (layer "F.Cu") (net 30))
 (segment (start 86.5 82.5) (end 87.5 82.5) (width 0.2) (layer "F.Cu") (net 30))
 (segment (start 150.951 96.901) (end 153.05 99) (width 0.2) (layer "F.Cu") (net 30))
 (segment (start 94.0339 82.601) (end 108.3339 96.901) (width 0.2) (layer "F.Cu") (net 30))
 (segment (start 92.399 82.601) (end 94.0339 82.601) (width 0.2) (layer "F.Cu") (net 30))
 (via (at 87.5 82.5) (size 0.6) (drill 0.3) (layers "F.Cu" "B.Cu") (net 30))
 (via (at 92.399 82.601) (size 0.6) (drill 0.3) (layers "F.Cu" "B.Cu") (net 30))
 (segment (start 92.5 82.5) (end 92.399 82.601) (width 0.2) (layer "B.Cu") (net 30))
 (segment (start 87.601 82.601) (end 92.399 82.601) (width 0.2) (layer "B.Cu") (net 30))
 (segment (start 87.5 82.5) (end 87.601 82.601) (width 0.2) (layer "B.Cu") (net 30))
 (segment (start 164.5 99) (end 171.55 99) (width 0.2) (layer "F.Cu") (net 31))
 (segment (start 94 82) (end 108.5 96.5) (width 0.2) (layer "F.Cu") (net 31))
 (segment (start 171.55 99) (end 180.45 99) (width 0.2) (layer "F.Cu") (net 31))
 (segment (start 87.12 79.41) (end 87.12 81.12) (width 0.2) (layer "F.Cu") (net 31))
 (segment (start 162 96.5) (end 164.5 99) (width 0.2) (layer "F.Cu") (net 31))
 (segment (start 91.5 82) (end 94 82) (width 0.2) (layer "F.Cu") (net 31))
 (segment (start 87.12 81.12) (end 87.5 81.5) (width 0.2) (layer "F.Cu") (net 31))
 (segment (start 108.5 96.5) (end 162 96.5) (width 0.2) (layer "F.Cu") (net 31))
 (via (at 87.5 81.5) (size 0.6) (drill 0.3) (layers "F.Cu" "B.Cu") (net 31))
 (via (at 91.5 82) (size 0.6) (drill 0.3) (layers "F.Cu" "B.Cu") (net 31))
 (segment (start 88 82) (end 91.5 82) (width 0.2) (layer "B.Cu") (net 31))
 (segment (start 87.5 81.5) (end 88 82) (width 0.2) (layer "B.Cu") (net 31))
 (segment (start 85 100.5) (end 86.549999 100.5) (width 0.2) (layer "F.Cu") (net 9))
 (segment (start 89.7 97.349999) (end 89.7 96.8375) (width 0.2) (layer "F.Cu") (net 9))
 (segment (start 88.597 88.097) (end 89 88.5) (width 0.2) (layer "F.Cu") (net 9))
 (segment (start 86.549999 100.5) (end 89.7 97.349999) (width 0.2) (layer "F.Cu") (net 9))
 (segment (start 89.66 63.335) (end 88.597 64.398) (width 0.2) (layer "F.Cu") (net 9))
 (segment (start 88.597 64.398) (end 88.597 88.097) (width 0.2) (layer "F.Cu") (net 9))
 (via (at 85 100.5) (size 0.6) (drill 0.3) (layers "F.Cu" "B.Cu") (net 9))
 (via (at 89 88.5) (size 0.6) (drill 0.3) (layers "F.Cu" "B.Cu") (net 9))
 (segment (start 89 96.5) (end 85 100.5) (width 0.2) (layer "B.Cu") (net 9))
 (segment (start 89 88.5) (end 89 96.5) (width 0.2) (layer "B.Cu") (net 9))
 (segment (start 82 98.5) (end 87.3875 98.5) (width 0.2) (layer "F.Cu") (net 8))
 (segment (start 90.723 64.812) (end 90.723 87.626943) (width 0.2) (layer "F.Cu") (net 8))
 (segment (start 87.3875 98.5) (end 89.05 96.8375) (width 0.2) (layer "F.Cu") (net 8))
 (segment (start 90.723 87.626943) (end 85.849943 92.5) (width 0.2) (layer "F.Cu") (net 8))
 (segment (start 92.2 63.335) (end 90.723 64.812) (width 0.2) (layer "F.Cu") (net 8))
 (segment (start 85.849943 92.5) (end 85.5 92.5) (width 0.2) (layer "F.Cu") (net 8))
 (via (at 82 98.5) (size 0.6) (drill 0.3) (layers "F.Cu" "B.Cu") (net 8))
 (via (at 85.5 92.5) (size 0.6) (drill 0.3) (layers "F.Cu" "B.Cu") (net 8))
 (segment (start 85.5 95) (end 82 98.5) (width 0.2) (layer "B.Cu") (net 8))
 (segment (start 85.5 92.5) (end 85.5 95) (width 0.2) (layer "B.Cu") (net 8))
 (segment (start 79.5 63.335) (end 78.437 64.398) (width 0.2) (layer "F.Cu") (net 5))
 (segment (start 78.437 86.286943) (end 86.800057 94.65) (width 0.2) (layer "F.Cu") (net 5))
 (segment (start 86.800057 94.65) (end 88.1625 94.65) (width 0.2) (layer "F.Cu") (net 5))
 (segment (start 78.437 64.398) (end 78.437 86.286943) (width 0.2) (layer "F.Cu") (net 5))
 (segment (start 113.804 65) (end 98.484626 65) (width 0.2) (layer "F.Cu") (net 32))
 (segment (start 84.58 62.25737) (end 84.58 63.335) (width 0.2) (layer "F.Cu") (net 32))
 (segment (start 170.73 59.5) (end 118.23 59.5) (width 0.2) (layer "F.Cu") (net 32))
 (segment (start 172.23 61) (end 170.73 59.5) (width 0.2) (layer "F.Cu") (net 32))
 (segment (start 98.484626 63.926) (end 95.541626 60.983) (width 0.2) (layer "F.Cu") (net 32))
 (segment (start 95.541626 60.983) (end 85.85437 60.983) (width 0.2) (layer "F.Cu") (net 32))
 (segment (start 85.85437 60.983) (end 84.58 62.25737) (width 0.2) (layer "F.Cu") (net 32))
 (segment (start 113.804 65) (end 113.804 63.926) (width 0.2) (layer "F.Cu") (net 32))
 (segment (start 118.23 59.5) (end 115.73 62) (width 0.2) (layer "F.Cu") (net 32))
 (segment (start 115.73 62) (end 113.804 63.926) (width 0.2) (layer "F.Cu") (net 32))
 (segment (start 98.484626 63.926) (end 98.484626 65) (width 0.2) (layer "F.Cu") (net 32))
 (segment (start 95 91.5) (end 95 91.933824) (width 0.2) (layer "F.Cu") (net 20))
 (segment (start 120.81 63.69) (end 109 75.5) (width 0.2) (layer "F.Cu") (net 20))
 (segment (start 120.81 62) (end 120.81 63.69) (width 0.2) (layer "F.Cu") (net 20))
 (segment (start 101 83.5) (end 100.5 83.5) (width 0.2) (layer "F.Cu") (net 20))
 (segment (start 107 77.5) (end 101 83.5) (width 0.2) (layer "F.Cu") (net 20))
 (segment (start 94.233824 92.7) (end 93.8375 92.7) (width 0.2) (layer "F.Cu") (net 20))
 (segment (start 109 75.5) (end 108.5 76) (width 0.2) (layer "F.Cu") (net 20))
 (segment (start 95 91.933824) (end 94.233824 92.7) (width 0.2) (layer "F.Cu") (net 20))
 (via (at 100.5 83.5) (size 0.6) (drill 0.3) (layers "F.Cu" "B.Cu") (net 20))
 (via (at 95 91.5) (size 0.6) (drill 0.3) (layers "F.Cu" "B.Cu") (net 20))
 (via (at 108.5 76) (size 0.6) (drill 0.3) (layers "F.Cu" "B.Cu") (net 20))
 (via (at 107 77.5) (size 0.6) (drill 0.3) (layers "F.Cu" "B.Cu") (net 20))
 (segment (start 100.5 86) (end 96.5 90) (width 0.2) (layer "B.Cu") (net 20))
 (segment (start 108.5 76) (end 107 77.5) (width 0.2) (layer "B.Cu") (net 20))
 (segment (start 100.5 83.5) (end 100.5 86) (width 0.2) (layer "B.Cu") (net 20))
 (segment (start 96.5 90) (end 95 91.5) (width 0.2) (layer "B.Cu") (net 20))
 (segment (start 96 91) (end 96 91.583824) (width 0.2) (layer "F.Cu") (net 19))
 (segment (start 100 82.5) (end 98.5 82.5) (width 0.2) (layer "F.Cu") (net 19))
 (segment (start 118.27 62) (end 118.27 64.23) (width 0.2) (layer "F.Cu") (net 19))
 (segment (start 94.233824 93.35) (end 93.8375 93.35) (width 0.2) (layer "F.Cu") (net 19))
 (segment (start 118.27 64.23) (end 108 74.5) (width 0.2) (layer "F.Cu") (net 19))
 (segment (start 96 91.583824) (end 94.233824 93.35) (width 0.2) (layer "F.Cu") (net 19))
 (segment (start 94.5 89.5) (end 96 91) (width 0.2) (layer "F.Cu") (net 19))
 (segment (start 105 77.5) (end 100 82.5) (width 0.2) (layer "F.Cu") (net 19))
 (via (at 108 74.5) (size 0.6) (drill 0.3) (layers "F.Cu" "B.Cu") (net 19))
 (via (at 105 77.5) (size 0.6) (drill 0.3) (layers "F.Cu" "B.Cu") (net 19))
 (via (at 98.5 82.5) (size 0.6) (drill 0.3) (layers "F.Cu" "B.Cu") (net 19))
 (via (at 94.5 89.5) (size 0.6) (drill 0.3) (layers "F.Cu" "B.Cu") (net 19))
 (segment (start 98.5 82.5) (end 98.5 85.849943) (width 0.2) (layer "B.Cu") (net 19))
 (segment (start 98.5 85.849943) (end 94.849943 89.5) (width 0.2) (layer "B.Cu") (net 19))
 (segment (start 108 74.5) (end 105 77.5) (width 0.2) (layer "B.Cu") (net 19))
 (segment (start 94.849943 89.5) (end 94.5 89.5) (width 0.2) (layer "B.Cu") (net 19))
 (segment (start 174.77 61) (end 175.971 59.799) (width 0.2) (layer "F.Cu") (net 17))
 (segment (start 175.971 59.799) (end 177.807471 59.799) (width 0.2) (layer "F.Cu") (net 17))
 (segment (start 94.349999 94.65) (end 93.8375 94.65) (width 0.2) (layer "F.Cu") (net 17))
 (segment (start 190.401 105.6661) (end 190.1661 105.901) (width 0.2) (layer "F.Cu") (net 17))
 (segment (start 190.401 72.392529) (end 190.401 105.6661) (width 0.2) (layer "F.Cu") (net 17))
 (segment (start 190.1661 105.901) (end 105.600999 105.901) (width 0.2) (layer "F.Cu") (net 17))
 (segment (start 177.807471 59.799) (end 190.401 72.392529) (width 0.2) (layer "F.Cu") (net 17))
 (segment (start 105.600999 105.901) (end 94.349999 94.65) (width 0.2) (layer "F.Cu") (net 17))
 (segment (start 94.349999 94) (end 93.8375 94) (width 0.2) (layer "F.Cu") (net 18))
 (segment (start 190 105.5) (end 105.849999 105.5) (width 0.2) (layer "F.Cu") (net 18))
 (segment (start 190 73.69) (end 190 105.5) (width 0.2) (layer "F.Cu") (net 18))
 (segment (start 105.849999 105.5) (end 94.349999 94) (width 0.2) (layer "F.Cu") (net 18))
 (segment (start 177.31 61) (end 190 73.69) (width 0.2) (layer "F.Cu") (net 18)))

